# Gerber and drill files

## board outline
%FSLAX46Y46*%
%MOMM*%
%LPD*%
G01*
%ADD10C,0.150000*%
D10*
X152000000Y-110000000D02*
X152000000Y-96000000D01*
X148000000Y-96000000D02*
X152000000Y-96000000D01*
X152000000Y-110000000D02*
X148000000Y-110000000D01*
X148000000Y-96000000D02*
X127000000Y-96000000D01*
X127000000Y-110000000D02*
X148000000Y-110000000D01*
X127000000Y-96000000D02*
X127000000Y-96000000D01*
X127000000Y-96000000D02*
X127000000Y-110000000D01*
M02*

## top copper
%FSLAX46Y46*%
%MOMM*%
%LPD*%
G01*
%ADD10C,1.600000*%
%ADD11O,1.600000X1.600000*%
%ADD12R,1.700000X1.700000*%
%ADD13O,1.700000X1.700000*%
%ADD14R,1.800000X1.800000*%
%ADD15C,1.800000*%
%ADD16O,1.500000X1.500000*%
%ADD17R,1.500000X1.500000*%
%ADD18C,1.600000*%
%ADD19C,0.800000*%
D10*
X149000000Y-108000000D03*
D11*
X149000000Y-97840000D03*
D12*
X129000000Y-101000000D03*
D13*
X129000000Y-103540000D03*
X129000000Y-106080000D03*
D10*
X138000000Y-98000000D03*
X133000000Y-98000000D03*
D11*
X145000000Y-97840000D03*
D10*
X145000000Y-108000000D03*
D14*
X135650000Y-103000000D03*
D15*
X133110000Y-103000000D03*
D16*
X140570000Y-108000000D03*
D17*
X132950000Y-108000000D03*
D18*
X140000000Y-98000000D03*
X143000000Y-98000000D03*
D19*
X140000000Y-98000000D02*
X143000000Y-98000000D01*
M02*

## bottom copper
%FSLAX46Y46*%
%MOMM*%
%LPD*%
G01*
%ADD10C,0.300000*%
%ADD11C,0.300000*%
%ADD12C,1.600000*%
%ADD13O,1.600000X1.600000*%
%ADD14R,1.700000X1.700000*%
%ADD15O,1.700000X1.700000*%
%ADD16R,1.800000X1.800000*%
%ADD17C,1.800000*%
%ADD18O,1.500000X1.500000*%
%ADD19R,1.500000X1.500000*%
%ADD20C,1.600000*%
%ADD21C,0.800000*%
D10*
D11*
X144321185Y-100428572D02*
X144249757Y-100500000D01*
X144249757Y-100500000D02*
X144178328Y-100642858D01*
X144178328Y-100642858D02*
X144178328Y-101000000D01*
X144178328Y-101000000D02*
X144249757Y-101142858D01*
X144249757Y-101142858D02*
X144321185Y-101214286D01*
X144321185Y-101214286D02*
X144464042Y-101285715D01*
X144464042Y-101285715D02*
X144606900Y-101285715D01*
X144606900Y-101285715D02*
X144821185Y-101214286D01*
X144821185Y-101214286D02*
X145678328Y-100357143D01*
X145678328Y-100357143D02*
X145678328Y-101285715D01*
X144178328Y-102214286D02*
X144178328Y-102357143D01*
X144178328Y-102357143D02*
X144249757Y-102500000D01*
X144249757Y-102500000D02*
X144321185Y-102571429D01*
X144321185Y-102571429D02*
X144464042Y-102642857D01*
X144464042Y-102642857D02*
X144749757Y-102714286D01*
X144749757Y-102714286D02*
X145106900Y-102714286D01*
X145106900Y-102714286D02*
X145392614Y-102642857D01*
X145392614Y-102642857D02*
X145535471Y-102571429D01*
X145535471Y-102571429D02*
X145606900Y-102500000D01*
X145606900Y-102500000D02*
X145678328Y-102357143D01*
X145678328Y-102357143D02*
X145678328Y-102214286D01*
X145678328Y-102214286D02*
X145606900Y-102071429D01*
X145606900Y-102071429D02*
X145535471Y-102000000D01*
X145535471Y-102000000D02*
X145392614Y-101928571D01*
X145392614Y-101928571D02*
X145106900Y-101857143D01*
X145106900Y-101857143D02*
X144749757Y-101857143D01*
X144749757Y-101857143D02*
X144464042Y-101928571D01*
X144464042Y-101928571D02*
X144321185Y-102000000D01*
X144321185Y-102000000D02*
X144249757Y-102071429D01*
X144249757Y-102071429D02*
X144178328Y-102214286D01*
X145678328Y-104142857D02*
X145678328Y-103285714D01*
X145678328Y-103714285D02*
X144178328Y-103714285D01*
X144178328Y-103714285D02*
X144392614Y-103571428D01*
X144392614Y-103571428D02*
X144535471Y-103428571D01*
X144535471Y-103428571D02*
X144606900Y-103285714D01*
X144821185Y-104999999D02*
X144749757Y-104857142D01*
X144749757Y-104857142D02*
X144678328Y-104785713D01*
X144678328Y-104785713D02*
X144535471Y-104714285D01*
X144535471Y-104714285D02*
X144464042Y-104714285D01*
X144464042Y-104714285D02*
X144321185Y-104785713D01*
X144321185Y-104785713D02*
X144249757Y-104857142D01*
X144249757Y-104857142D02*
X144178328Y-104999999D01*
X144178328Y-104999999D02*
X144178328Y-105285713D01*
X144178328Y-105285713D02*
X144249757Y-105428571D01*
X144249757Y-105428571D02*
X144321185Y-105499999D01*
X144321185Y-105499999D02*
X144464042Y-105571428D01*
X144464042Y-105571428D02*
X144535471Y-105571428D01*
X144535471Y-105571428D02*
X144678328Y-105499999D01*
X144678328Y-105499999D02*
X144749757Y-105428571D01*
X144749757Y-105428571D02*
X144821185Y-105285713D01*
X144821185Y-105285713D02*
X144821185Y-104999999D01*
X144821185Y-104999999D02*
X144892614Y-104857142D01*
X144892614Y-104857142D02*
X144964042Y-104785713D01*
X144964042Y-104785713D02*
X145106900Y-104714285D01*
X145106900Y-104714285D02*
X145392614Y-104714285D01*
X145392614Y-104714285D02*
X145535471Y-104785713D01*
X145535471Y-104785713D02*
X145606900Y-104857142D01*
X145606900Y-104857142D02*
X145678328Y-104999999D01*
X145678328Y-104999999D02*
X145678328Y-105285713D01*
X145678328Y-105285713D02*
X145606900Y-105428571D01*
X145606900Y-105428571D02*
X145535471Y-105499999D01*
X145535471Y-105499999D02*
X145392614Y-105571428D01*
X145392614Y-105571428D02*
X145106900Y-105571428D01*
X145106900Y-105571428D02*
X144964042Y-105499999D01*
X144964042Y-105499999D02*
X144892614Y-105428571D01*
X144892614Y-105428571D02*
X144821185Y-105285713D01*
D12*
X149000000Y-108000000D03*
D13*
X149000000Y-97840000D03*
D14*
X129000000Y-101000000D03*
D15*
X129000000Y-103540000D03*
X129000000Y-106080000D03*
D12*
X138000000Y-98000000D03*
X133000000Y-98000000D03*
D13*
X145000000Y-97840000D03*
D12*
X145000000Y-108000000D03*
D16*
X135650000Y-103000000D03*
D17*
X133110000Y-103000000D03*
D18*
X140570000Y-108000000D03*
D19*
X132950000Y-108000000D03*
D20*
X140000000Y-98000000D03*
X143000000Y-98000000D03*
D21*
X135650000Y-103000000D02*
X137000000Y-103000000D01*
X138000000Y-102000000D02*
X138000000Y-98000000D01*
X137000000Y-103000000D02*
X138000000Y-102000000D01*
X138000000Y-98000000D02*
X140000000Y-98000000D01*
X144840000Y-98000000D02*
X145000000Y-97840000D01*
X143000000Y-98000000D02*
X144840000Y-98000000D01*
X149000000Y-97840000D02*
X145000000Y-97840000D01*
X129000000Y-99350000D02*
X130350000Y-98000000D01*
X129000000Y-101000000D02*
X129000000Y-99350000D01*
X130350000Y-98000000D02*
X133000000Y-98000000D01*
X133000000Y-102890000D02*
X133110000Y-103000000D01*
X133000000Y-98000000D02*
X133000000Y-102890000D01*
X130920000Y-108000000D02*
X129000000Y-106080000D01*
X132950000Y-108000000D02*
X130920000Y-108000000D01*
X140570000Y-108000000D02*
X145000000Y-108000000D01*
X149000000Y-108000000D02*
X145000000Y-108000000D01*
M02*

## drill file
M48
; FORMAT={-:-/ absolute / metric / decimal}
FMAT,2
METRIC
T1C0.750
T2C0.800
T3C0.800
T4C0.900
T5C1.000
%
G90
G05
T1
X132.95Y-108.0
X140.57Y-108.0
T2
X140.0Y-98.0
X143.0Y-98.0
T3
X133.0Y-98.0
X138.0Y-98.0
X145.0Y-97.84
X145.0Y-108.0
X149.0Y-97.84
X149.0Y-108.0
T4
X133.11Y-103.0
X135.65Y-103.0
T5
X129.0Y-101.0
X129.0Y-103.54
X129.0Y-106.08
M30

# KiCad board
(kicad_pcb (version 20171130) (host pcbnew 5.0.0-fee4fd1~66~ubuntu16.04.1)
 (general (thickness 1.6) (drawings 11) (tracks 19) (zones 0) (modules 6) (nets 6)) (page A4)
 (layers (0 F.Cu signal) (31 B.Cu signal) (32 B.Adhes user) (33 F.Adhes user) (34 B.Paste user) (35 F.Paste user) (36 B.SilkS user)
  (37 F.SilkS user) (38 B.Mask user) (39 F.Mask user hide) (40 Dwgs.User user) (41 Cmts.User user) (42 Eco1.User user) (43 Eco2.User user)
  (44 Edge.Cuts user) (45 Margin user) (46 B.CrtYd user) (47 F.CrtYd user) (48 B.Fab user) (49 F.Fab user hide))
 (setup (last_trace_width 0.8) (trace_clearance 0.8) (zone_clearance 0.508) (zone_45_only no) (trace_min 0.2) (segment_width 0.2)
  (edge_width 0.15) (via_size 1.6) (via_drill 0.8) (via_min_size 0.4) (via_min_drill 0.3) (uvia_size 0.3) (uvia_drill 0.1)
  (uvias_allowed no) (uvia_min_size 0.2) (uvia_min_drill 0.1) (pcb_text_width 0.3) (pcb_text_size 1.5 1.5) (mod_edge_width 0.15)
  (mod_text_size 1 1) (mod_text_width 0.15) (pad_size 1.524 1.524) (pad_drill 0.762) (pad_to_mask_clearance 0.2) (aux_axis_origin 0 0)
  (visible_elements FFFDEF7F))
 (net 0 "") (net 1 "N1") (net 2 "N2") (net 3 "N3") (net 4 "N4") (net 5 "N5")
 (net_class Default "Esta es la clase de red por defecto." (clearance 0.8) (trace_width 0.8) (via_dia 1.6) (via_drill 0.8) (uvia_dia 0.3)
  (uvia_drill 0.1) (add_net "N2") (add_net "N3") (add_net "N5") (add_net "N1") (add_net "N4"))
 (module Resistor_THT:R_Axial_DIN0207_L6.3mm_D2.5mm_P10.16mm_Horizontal (layer F.Cu) (at 149 108 90)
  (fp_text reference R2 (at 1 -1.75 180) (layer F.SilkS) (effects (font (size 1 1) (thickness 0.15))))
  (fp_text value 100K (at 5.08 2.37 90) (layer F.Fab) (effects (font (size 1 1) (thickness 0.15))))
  (pad 1 thru_hole circle (at 0 0 90) (size 1.6 1.6) (drill 0.8) (layers *.Cu *.Mask) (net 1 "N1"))
  (pad 2 thru_hole oval (at 10.16 0 90) (size 1.6 1.6) (drill 0.8) (layers *.Cu *.Mask) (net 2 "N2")))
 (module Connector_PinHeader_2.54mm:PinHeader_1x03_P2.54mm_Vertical (layer F.Cu) (at 129 101)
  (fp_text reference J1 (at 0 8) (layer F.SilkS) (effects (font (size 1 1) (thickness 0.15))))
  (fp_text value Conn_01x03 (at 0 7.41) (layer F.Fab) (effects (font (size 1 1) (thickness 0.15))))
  (pad 1 thru_hole rect (at 0 0) (size 1.7 1.7) (drill 1) (layers *.Cu *.Mask) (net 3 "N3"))
  (pad 2 thru_hole oval (at 0 2.54) (size 1.7 1.7) (drill 1) (layers *.Cu *.Mask) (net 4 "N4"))
  (pad 3 thru_hole oval (at 0 5.08) (size 1.7 1.7) (drill 1) (layers *.Cu *.Mask) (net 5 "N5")))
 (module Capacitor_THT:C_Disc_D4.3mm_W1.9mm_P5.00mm (layer F.Cu) (at 138 98 180)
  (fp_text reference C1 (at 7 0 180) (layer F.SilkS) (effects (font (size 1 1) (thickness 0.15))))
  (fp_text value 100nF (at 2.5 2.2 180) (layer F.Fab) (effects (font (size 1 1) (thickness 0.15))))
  (pad 1 thru_hole circle (at 0 0 180) (size 1.6 1.6) (drill 0.8) (layers *.Cu *.Mask) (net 2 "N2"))
  (pad 2 thru_hole circle (at 5 0 180) (size 1.6 1.6) (drill 0.8) (layers *.Cu *.Mask) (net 3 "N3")))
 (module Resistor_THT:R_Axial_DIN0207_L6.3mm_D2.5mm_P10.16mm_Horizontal (layer F.Cu) (at 145 108 90)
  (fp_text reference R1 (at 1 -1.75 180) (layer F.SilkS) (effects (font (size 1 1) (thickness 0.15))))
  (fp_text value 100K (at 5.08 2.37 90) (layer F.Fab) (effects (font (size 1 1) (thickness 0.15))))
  (pad 2 thru_hole oval (at 10.16 0 90) (size 1.6 1.6) (drill 0.8) (layers *.Cu *.Mask) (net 2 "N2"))
  (pad 1 thru_hole circle (at 0 0 90) (size 1.6 1.6) (drill 0.8) (layers *.Cu *.Mask) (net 1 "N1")))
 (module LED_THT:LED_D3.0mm (layer F.Cu) (at 135.65 103 180) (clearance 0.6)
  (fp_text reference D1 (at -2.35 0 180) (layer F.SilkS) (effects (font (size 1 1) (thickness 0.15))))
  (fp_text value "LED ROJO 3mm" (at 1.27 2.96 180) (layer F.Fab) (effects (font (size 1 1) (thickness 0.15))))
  (pad 1 thru_hole rect (at 0 0 180) (size 1.8 1.8) (drill 0.9) (layers *.Cu *.Mask) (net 2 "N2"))
  (pad 2 thru_hole circle (at 2.54 0 180) (size 1.8 1.8) (drill 0.9) (layers *.Cu *.Mask) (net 3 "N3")))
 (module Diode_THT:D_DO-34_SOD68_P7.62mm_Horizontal (layer F.Cu) (at 132.95 108)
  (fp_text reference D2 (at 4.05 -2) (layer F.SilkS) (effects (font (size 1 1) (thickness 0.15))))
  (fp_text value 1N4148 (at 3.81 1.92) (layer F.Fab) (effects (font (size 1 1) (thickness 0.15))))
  (pad 2 thru_hole oval (at 7.62 0) (size 1.5 1.5) (drill 0.75) (layers *.Cu *.Mask) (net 1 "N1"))
  (pad 1 thru_hole rect (at 0 0) (size 1.5 1.5) (drill 0.75) (layers *.Cu *.Mask) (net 5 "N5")))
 (gr_line (start 152 110) (end 152 96) (layer Edge.Cuts) (width 0.15))
 (gr_line (start 148 96) (end 152 96) (layer Edge.Cuts) (width 0.15))
 (gr_line (start 152 110) (end 148 110) (layer Edge.Cuts) (width 0.15))
 (gr_line (start 148 96) (end 127 96) (layer Edge.Cuts) (width 0.15))
 (gr_line (start 127 110) (end 148 110) (layer Edge.Cuts) (width 0.15))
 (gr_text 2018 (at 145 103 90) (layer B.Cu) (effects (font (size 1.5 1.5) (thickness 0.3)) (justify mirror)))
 (gr_line (start 127 96) (end 127 96) (layer Edge.Cuts) (width 0.15))
 (gr_line (start 127 96) (end 127 110) (layer Edge.Cuts) (width 0.15))
 (segment (start 135.65 103) (end 137 103) (width 0.8) (layer B.Cu) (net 2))
 (segment (start 138 102) (end 138 98) (width 0.8) (layer B.Cu) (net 2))
 (segment (start 137 103) (end 138 102) (width 0.8) (layer B.Cu) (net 2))
 (via (at 140 98) (size 1.6) (drill 0.8) (layers F.Cu B.Cu) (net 2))
 (segment (start 138 98) (end 140 98) (width 0.8) (layer B.Cu) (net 2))
 (via (at 143 98) (size 1.6) (drill 0.8) (layers F.Cu B.Cu) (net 2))
 (segment (start 140 98) (end 143 98) (width 0.8) (layer F.Cu) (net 2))
 (segment (start 144.84 98) (end 145 97.84) (width 0.8) (layer B.Cu) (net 2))
 (segment (start 143 98) (end 144.84 98) (width 0.8) (layer B.Cu) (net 2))
 (segment (start 149 97.84) (end 145 97.84) (width 0.8) (layer B.Cu) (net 2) (status 10))
 (segment (start 129 99.35) (end 130.35 98) (width 0.8) (layer B.Cu) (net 3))
 (segment (start 129 101) (end 129 99.35) (width 0.8) (layer B.Cu) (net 3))
 (segment (start 130.35 98) (end 133 98) (width 0.8) (layer B.Cu) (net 3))
 (segment (start 133 102.89) (end 133.11 103) (width 0.8) (layer B.Cu) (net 3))
 (segment (start 133 98) (end 133 102.89) (width 0.8) (layer B.Cu) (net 3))
 (segment (start 130.92 108) (end 129 106.08) (width 0.8) (layer B.Cu) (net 5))
 (segment (start 132.95 108) (end 130.92 108) (width 0.8) (layer B.Cu) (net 5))
 (segment (start 140.57 108) (end 145 108) (width 0.8) (layer B.Cu) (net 1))
 (segment (start 149 108) (end 145 108) (width 0.8) (layer B.Cu) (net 1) (status 10)))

